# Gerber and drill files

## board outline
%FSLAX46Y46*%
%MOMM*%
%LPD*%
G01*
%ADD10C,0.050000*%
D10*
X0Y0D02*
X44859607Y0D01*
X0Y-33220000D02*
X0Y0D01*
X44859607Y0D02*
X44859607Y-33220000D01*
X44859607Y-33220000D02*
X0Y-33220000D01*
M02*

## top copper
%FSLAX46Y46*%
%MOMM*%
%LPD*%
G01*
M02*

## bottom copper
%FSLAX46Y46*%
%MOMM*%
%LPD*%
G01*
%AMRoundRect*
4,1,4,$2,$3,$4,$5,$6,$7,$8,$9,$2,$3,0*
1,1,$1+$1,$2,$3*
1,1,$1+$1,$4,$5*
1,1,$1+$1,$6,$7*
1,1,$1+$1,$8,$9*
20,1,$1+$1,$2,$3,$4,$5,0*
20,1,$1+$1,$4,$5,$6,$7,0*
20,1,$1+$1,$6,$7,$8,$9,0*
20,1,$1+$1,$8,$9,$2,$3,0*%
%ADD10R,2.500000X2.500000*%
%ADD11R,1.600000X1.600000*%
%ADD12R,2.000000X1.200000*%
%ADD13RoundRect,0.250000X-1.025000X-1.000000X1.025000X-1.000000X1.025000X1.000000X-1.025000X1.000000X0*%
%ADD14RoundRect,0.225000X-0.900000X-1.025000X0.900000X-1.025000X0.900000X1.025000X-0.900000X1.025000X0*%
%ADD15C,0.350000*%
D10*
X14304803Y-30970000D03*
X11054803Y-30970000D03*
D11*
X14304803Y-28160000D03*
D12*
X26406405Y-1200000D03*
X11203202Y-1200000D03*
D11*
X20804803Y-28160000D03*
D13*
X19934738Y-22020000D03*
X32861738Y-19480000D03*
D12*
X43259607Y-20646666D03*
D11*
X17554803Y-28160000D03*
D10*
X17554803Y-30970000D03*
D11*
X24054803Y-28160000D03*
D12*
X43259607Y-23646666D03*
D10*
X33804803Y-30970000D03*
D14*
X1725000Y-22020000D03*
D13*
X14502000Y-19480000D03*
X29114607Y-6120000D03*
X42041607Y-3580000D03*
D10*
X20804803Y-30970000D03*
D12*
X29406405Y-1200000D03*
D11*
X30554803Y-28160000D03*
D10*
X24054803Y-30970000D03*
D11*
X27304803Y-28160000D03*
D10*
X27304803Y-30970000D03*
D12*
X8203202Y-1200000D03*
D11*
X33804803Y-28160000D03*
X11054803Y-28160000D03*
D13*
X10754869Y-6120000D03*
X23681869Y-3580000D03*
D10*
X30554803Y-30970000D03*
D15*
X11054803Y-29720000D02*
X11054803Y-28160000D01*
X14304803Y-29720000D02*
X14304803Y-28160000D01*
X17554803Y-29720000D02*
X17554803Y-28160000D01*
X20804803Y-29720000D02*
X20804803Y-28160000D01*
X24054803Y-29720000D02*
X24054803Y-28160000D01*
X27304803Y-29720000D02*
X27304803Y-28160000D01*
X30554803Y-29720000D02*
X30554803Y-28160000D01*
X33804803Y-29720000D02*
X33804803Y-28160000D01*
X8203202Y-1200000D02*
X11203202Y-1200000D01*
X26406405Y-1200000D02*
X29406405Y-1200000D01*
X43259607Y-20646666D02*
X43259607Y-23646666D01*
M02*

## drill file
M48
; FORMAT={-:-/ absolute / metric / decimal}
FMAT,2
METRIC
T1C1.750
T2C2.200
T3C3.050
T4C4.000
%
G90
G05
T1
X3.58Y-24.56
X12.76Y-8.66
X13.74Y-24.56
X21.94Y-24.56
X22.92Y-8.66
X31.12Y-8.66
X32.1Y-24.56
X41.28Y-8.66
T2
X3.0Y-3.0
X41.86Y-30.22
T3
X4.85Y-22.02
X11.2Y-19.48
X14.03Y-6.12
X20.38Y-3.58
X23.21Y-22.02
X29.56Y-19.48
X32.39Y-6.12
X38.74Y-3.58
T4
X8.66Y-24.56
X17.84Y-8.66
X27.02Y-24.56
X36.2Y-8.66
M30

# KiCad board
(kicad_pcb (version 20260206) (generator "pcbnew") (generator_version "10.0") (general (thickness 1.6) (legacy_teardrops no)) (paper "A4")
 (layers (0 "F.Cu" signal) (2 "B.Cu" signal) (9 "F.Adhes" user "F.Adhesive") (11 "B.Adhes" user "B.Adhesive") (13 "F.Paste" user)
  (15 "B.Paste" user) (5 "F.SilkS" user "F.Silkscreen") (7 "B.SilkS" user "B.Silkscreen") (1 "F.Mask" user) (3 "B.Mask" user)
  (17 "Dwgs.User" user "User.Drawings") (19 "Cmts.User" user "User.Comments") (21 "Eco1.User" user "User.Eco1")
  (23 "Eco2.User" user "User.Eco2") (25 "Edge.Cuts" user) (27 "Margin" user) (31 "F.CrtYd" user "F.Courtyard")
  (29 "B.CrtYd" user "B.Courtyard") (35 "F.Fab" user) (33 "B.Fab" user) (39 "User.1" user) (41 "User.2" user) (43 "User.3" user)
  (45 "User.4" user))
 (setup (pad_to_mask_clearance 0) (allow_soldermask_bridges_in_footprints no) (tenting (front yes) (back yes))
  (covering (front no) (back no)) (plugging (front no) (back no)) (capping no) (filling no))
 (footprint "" (layer "F.Cu") (at 0 0)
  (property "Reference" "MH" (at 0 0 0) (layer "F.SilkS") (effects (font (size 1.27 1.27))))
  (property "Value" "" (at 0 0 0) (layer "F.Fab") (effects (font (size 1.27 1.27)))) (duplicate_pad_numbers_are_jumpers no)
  (pad "" np_thru_hole circle (at 41.859607 30.22) (size 2.2 2.2) (drill 2.2) (layers "*.Cu")))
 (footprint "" (layer "F.Cu") (at 0 0)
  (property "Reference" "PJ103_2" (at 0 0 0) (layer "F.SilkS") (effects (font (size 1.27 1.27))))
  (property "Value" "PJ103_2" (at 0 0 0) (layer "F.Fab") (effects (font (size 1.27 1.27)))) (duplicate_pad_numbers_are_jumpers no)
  (pad "1" smd rect (at 14.304803 30.97) (size 2.5 2.5) (layers "B.Cu" "B.Mask") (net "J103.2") (thermal_bridge_angle 45)))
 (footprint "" (layer "F.Cu") (at 0 0)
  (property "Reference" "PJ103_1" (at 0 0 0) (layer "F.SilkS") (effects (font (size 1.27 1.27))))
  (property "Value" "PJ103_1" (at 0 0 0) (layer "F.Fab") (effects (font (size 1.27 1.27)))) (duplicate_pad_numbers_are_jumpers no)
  (pad "1" smd rect (at 11.054803 30.97) (size 2.5 2.5) (layers "B.Cu" "B.Mask") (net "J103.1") (thermal_bridge_angle 45)))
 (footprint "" (layer "F.Cu") (at 0 0)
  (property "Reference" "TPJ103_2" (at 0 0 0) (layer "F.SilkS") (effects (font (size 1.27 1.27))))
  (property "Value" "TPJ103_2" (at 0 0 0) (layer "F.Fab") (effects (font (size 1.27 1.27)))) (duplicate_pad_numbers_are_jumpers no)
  (pad "1" smd rect (at 14.304803 28.16) (size 1.6 1.6) (layers "B.Cu" "B.Mask") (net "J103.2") (thermal_bridge_angle 45)))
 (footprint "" (layer "F.Cu") (at 0 0)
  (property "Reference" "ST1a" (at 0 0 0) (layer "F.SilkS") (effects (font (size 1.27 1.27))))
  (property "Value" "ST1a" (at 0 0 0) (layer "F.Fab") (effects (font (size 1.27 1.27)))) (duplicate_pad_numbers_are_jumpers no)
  (pad "1" smd rect (at 26.406405 1.2) (size 2 1.2) (layers "B.Cu" "B.Mask") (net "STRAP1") (thermal_bridge_angle 45)))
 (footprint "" (layer "F.Cu") (at 0 0)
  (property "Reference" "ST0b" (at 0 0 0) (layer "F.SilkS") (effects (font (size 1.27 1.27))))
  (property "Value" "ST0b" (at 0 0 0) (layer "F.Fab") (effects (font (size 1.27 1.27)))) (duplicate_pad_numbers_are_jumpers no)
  (pad "1" smd rect (at 11.203202 1.2) (size 2 1.2) (layers "B.Cu" "B.Mask") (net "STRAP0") (thermal_bridge_angle 45)))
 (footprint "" (layer "F.Cu") (at 0 0)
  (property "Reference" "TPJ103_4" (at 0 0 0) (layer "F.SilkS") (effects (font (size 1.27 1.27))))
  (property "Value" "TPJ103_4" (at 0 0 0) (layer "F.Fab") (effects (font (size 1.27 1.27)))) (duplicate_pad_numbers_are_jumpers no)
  (pad "1" smd rect (at 20.804803 28.16) (size 1.6 1.6) (layers "B.Cu" "B.Mask") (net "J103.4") (thermal_bridge_angle 45)))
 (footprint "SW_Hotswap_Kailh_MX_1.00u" (layer "F.Cu") (at 27.019738 24.56)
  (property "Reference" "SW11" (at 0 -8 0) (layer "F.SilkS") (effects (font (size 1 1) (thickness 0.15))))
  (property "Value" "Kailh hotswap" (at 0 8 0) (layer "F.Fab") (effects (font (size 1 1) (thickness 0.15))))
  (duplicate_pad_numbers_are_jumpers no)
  (pad "" np_thru_hole circle (at -5.08 0) (size 1.75 1.75) (drill 1.75) (layers "*.Cu" "*.Mask"))
  (pad "" np_thru_hole circle (at -3.81 -2.54) (size 3.05 3.05) (drill 3.05) (layers "*.Cu" "*.Mask"))
  (pad "" np_thru_hole circle (at 0 0) (size 4 4) (drill 4) (layers "*.Cu" "*.Mask"))
  (pad "" np_thru_hole circle (at 2.54 -5.08) (size 3.05 3.05) (drill 3.05) (layers "*.Cu" "*.Mask"))
  (pad "" np_thru_hole circle (at 5.08 0) (size 1.75 1.75) (drill 1.75) (layers "*.Cu" "*.Mask"))
  (pad "1" smd roundrect (at -7.085 -2.54) (size 2.55 2.5) (layers "B.Cu" "B.Mask" "B.Paste") (roundrect_rratio 0.1) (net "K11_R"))
  (pad "2" smd roundrect (at 5.842 -5.08) (size 2.55 2.5) (layers "B.Cu" "B.Mask" "B.Paste") (roundrect_rratio 0.1) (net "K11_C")))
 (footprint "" (layer "F.Cu") (at 0 0)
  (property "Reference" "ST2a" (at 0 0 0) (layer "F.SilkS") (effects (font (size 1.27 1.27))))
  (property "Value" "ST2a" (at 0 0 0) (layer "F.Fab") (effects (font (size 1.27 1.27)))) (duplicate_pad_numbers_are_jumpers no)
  (pad "1" smd rect (at 43.259607 20.646666) (size 2 1.2) (layers "B.Cu" "B.Mask") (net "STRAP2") (thermal_bridge_angle 45)))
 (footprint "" (layer "F.Cu") (at 0 0)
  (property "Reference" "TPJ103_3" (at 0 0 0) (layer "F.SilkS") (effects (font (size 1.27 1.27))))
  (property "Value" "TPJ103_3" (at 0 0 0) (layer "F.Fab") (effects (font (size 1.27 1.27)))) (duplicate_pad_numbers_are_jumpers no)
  (pad "1" smd rect (at 17.554803 28.16) (size 1.6 1.6) (layers "B.Cu" "B.Mask") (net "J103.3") (thermal_bridge_angle 45)))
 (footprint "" (layer "F.Cu") (at 0 0)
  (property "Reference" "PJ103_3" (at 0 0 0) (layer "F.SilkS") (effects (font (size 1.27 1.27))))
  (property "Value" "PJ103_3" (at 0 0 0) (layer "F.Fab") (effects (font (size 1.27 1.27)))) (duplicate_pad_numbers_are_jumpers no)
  (pad "1" smd rect (at 17.554803 30.97) (size 2.5 2.5) (layers "B.Cu" "B.Mask") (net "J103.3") (thermal_bridge_angle 45)))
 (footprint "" (layer "F.Cu") (at 0 0)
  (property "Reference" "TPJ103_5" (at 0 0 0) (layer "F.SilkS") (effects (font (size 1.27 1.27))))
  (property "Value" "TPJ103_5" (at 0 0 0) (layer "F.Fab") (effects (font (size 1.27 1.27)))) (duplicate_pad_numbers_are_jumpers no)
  (pad "1" smd rect (at 24.054803 28.16) (size 1.6 1.6) (layers "B.Cu" "B.Mask") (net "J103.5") (thermal_bridge_angle 45)))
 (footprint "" (layer "F.Cu") (at 0 0)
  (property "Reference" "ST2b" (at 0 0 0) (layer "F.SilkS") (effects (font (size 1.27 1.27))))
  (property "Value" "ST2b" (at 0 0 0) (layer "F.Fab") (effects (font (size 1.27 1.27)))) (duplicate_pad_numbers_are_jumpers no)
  (pad "1" smd rect (at 43.259607 23.646666) (size 2 1.2) (layers "B.Cu" "B.Mask") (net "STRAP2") (thermal_bridge_angle 45)))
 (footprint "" (layer "F.Cu") (at 0 0)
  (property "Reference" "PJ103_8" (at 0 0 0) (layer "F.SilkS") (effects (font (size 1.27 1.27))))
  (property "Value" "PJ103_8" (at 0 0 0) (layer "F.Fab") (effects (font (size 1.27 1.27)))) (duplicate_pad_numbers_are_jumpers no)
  (pad "1" smd rect (at 33.804803 30.97) (size 2.5 2.5) (layers "B.Cu" "B.Mask") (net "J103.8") (thermal_bridge_angle 45)))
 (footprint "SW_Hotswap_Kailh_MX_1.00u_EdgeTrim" (layer "F.Cu") (at 8.66 24.56)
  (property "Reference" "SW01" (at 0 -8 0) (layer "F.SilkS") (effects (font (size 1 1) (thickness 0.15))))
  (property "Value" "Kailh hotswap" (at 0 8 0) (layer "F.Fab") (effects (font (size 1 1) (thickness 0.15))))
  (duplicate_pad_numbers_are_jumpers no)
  (pad "" np_thru_hole circle (at -5.08 0) (size 1.75 1.75) (drill 1.75) (layers "*.Cu" "*.Mask"))
  (pad "" np_thru_hole circle (at -3.81 -2.54) (size 3.05 3.05) (drill 3.05) (layers "*.Cu" "*.Mask"))
  (pad "" np_thru_hole circle (at 0 0) (size 4 4) (drill 4) (layers "*.Cu" "*.Mask"))
  (pad "" np_thru_hole circle (at 2.54 -5.08) (size 3.05 3.05) (drill 3.05) (layers "*.Cu" "*.Mask"))
  (pad "" np_thru_hole circle (at 5.08 0) (size 1.75 1.75) (drill 1.75) (layers "*.Cu" "*.Mask"))
  (pad "1" smd roundrect (at -6.935 -2.54) (size 2.25 2.5) (layers "B.Cu" "B.Mask" "B.Paste") (roundrect_rratio 0.1) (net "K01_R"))
  (pad "2" smd roundrect (at 5.842 -5.08) (size 2.55 2.5) (layers "B.Cu" "B.Mask" "B.Paste") (roundrect_rratio 0.1) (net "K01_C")))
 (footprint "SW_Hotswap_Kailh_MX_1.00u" (layer "F.Cu") (at 36.199607 8.66)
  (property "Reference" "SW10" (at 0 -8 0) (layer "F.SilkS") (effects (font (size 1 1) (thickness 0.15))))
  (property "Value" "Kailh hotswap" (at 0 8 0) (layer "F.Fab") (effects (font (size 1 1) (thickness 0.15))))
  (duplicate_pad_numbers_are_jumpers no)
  (pad "" np_thru_hole circle (at -5.08 0) (size 1.75 1.75) (drill 1.75) (layers "*.Cu" "*.Mask"))
  (pad "" np_thru_hole circle (at -3.81 -2.54) (size 3.05 3.05) (drill 3.05) (layers "*.Cu" "*.Mask"))
  (pad "" np_thru_hole circle (at 0 0) (size 4 4) (drill 4) (layers "*.Cu" "*.Mask"))
  (pad "" np_thru_hole circle (at 2.54 -5.08) (size 3.05 3.05) (drill 3.05) (layers "*.Cu" "*.Mask"))
  (pad "" np_thru_hole circle (at 5.08 0) (size 1.75 1.75) (drill 1.75) (layers "*.Cu" "*.Mask"))
  (pad "1" smd roundrect (at -7.085 -2.54) (size 2.55 2.5) (layers "B.Cu" "B.Mask" "B.Paste") (roundrect_rratio 0.1) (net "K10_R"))
  (pad "2" smd roundrect (at 5.842 -5.08) (size 2.55 2.5) (layers "B.Cu" "B.Mask" "B.Paste") (roundrect_rratio 0.1) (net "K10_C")))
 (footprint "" (layer "F.Cu") (at 0 0)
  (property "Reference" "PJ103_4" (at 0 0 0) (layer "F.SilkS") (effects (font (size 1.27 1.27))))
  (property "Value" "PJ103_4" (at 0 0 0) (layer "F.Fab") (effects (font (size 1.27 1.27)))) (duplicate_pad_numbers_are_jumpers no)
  (pad "1" smd rect (at 20.804803 30.97) (size 2.5 2.5) (layers "B.Cu" "B.Mask") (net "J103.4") (thermal_bridge_angle 45)))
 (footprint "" (layer "F.Cu") (at 0 0)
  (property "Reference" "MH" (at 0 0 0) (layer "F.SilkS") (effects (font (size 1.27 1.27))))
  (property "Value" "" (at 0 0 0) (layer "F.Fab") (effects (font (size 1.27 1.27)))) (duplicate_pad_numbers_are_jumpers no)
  (pad "" np_thru_hole circle (at 3 3) (size 2.2 2.2) (drill 2.2) (layers "*.Cu")))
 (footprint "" (layer "F.Cu") (at 0 0)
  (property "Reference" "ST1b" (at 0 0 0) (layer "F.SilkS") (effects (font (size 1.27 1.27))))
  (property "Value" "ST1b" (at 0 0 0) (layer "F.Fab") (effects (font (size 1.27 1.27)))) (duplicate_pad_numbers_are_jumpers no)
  (pad "1" smd rect (at 29.406405 1.2) (size 2 1.2) (layers "B.Cu" "B.Mask") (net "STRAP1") (thermal_bridge_angle 45)))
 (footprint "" (layer "F.Cu") (at 0 0)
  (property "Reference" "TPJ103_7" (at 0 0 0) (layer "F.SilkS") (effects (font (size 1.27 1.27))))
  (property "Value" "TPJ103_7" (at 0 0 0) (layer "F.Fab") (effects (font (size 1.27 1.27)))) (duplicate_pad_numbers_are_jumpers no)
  (pad "1" smd rect (at 30.554803 28.16) (size 1.6 1.6) (layers "B.Cu" "B.Mask") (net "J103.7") (thermal_bridge_angle 45)))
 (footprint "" (layer "F.Cu") (at 0 0)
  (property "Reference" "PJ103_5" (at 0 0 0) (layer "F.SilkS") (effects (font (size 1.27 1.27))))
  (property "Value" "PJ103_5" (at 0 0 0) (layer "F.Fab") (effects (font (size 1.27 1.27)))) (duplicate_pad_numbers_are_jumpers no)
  (pad "1" smd rect (at 24.054803 30.97) (size 2.5 2.5) (layers "B.Cu" "B.Mask") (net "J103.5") (thermal_bridge_angle 45)))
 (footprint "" (layer "F.Cu") (at 0 0)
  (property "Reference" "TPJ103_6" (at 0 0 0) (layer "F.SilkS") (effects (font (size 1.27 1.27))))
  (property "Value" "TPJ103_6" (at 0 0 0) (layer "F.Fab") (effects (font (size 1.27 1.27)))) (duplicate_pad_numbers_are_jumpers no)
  (pad "1" smd rect (at 27.304803 28.16) (size 1.6 1.6) (layers "B.Cu" "B.Mask") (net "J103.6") (thermal_bridge_angle 45)))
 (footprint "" (layer "F.Cu") (at 0 0)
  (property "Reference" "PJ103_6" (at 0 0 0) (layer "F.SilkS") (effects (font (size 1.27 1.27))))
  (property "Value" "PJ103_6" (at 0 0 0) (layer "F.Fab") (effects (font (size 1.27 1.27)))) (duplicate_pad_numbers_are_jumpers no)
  (pad "1" smd rect (at 27.304803 30.97) (size 2.5 2.5) (layers "B.Cu" "B.Mask") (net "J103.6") (thermal_bridge_angle 45)))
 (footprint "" (layer "F.Cu") (at 0 0)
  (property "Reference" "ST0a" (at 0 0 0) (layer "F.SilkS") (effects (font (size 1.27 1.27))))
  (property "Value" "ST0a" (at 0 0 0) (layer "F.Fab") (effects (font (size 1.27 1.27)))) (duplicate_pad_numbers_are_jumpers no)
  (pad "1" smd rect (at 8.203202 1.2) (size 2 1.2) (layers "B.Cu" "B.Mask") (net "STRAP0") (thermal_bridge_angle 45)))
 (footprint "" (layer "F.Cu") (at 0 0)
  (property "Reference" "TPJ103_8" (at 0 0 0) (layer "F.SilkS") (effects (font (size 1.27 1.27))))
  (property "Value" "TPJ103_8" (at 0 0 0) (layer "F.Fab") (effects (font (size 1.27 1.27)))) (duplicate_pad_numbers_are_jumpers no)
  (pad "1" smd rect (at 33.804803 28.16) (size 1.6 1.6) (layers "B.Cu" "B.Mask") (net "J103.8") (thermal_bridge_angle 45)))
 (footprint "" (layer "F.Cu") (at 0 0)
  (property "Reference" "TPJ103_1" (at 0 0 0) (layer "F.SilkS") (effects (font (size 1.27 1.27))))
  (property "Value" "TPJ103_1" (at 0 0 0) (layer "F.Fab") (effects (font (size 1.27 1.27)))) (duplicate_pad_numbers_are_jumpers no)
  (pad "1" smd rect (at 11.054803 28.16) (size 1.6 1.6) (layers "B.Cu" "B.Mask") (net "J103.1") (thermal_bridge_angle 45)))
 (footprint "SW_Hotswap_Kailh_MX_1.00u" (layer "F.Cu") (at 17.839869 8.66)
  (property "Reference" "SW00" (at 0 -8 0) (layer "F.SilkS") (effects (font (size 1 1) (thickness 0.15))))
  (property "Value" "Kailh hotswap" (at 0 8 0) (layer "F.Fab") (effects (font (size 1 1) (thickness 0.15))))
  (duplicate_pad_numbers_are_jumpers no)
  (pad "" np_thru_hole circle (at -5.08 0) (size 1.75 1.75) (drill 1.75) (layers "*.Cu" "*.Mask"))
  (pad "" np_thru_hole circle (at -3.81 -2.54) (size 3.05 3.05) (drill 3.05) (layers "*.Cu" "*.Mask"))
  (pad "" np_thru_hole circle (at 0 0) (size 4 4) (drill 4) (layers "*.Cu" "*.Mask"))
  (pad "" np_thru_hole circle (at 2.54 -5.08) (size 3.05 3.05) (drill 3.05) (layers "*.Cu" "*.Mask"))
  (pad "" np_thru_hole circle (at 5.08 0) (size 1.75 1.75) (drill 1.75) (layers "*.Cu" "*.Mask"))
  (pad "1" smd roundrect (at -7.085 -2.54) (size 2.55 2.5) (layers "B.Cu" "B.Mask" "B.Paste") (roundrect_rratio 0.1) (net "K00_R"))
  (pad "2" smd roundrect (at 5.842 -5.08) (size 2.55 2.5) (layers "B.Cu" "B.Mask" "B.Paste") (roundrect_rratio 0.1) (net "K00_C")))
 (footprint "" (layer "F.Cu") (at 0 0)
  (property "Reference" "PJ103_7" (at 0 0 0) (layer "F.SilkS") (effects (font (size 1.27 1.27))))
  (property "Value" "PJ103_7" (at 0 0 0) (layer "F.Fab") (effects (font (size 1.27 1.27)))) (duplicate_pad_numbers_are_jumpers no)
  (pad "1" smd rect (at 30.554803 30.97) (size 2.5 2.5) (layers "B.Cu" "B.Mask") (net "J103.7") (thermal_bridge_angle 45)))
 (gr_line (start 0 0) (end 44.859607 0) (stroke (width 0.05) (type default)) (layer "Edge.Cuts"))
 (gr_line (start 0 33.22) (end 0 0) (stroke (width 0.05) (type default)) (layer "Edge.Cuts"))
 (gr_line (start 44.859607 0) (end 44.859607 33.22) (stroke (width 0.05) (type default)) (layer "Edge.Cuts"))
 (gr_line (start 44.859607 33.22) (end 0 33.22) (stroke (width 0.05) (type default)) (layer "Edge.Cuts"))
 (segment (start 11.054803 29.72) (end 11.054803 28.16) (width 0.35) (layer "B.Cu") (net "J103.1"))
 (segment (start 14.304803 29.72) (end 14.304803 28.16) (width 0.35) (layer "B.Cu") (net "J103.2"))
 (segment (start 17.554803 29.72) (end 17.554803 28.16) (width 0.35) (layer "B.Cu") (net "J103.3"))
 (segment (start 20.804803 29.72) (end 20.804803 28.16) (width 0.35) (layer "B.Cu") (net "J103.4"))
 (segment (start 24.054803 29.72) (end 24.054803 28.16) (width 0.35) (layer "B.Cu") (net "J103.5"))
 (segment (start 27.304803 29.72) (end 27.304803 28.16) (width 0.35) (layer "B.Cu") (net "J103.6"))
 (segment (start 30.554803 29.72) (end 30.554803 28.16) (width 0.35) (layer "B.Cu") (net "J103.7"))
 (segment (start 33.804803 29.72) (end 33.804803 28.16) (width 0.35) (layer "B.Cu") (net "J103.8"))
 (segment (start 8.203202 1.2) (end 11.203202 1.2) (width 0.35) (layer "B.Cu") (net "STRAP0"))
 (segment (start 26.406405 1.2) (end 29.406405 1.2) (width 0.35) (layer "B.Cu") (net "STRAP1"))
 (segment (start 43.259607 20.646666) (end 43.259607 23.646666) (width 0.35) (layer "B.Cu") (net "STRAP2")))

